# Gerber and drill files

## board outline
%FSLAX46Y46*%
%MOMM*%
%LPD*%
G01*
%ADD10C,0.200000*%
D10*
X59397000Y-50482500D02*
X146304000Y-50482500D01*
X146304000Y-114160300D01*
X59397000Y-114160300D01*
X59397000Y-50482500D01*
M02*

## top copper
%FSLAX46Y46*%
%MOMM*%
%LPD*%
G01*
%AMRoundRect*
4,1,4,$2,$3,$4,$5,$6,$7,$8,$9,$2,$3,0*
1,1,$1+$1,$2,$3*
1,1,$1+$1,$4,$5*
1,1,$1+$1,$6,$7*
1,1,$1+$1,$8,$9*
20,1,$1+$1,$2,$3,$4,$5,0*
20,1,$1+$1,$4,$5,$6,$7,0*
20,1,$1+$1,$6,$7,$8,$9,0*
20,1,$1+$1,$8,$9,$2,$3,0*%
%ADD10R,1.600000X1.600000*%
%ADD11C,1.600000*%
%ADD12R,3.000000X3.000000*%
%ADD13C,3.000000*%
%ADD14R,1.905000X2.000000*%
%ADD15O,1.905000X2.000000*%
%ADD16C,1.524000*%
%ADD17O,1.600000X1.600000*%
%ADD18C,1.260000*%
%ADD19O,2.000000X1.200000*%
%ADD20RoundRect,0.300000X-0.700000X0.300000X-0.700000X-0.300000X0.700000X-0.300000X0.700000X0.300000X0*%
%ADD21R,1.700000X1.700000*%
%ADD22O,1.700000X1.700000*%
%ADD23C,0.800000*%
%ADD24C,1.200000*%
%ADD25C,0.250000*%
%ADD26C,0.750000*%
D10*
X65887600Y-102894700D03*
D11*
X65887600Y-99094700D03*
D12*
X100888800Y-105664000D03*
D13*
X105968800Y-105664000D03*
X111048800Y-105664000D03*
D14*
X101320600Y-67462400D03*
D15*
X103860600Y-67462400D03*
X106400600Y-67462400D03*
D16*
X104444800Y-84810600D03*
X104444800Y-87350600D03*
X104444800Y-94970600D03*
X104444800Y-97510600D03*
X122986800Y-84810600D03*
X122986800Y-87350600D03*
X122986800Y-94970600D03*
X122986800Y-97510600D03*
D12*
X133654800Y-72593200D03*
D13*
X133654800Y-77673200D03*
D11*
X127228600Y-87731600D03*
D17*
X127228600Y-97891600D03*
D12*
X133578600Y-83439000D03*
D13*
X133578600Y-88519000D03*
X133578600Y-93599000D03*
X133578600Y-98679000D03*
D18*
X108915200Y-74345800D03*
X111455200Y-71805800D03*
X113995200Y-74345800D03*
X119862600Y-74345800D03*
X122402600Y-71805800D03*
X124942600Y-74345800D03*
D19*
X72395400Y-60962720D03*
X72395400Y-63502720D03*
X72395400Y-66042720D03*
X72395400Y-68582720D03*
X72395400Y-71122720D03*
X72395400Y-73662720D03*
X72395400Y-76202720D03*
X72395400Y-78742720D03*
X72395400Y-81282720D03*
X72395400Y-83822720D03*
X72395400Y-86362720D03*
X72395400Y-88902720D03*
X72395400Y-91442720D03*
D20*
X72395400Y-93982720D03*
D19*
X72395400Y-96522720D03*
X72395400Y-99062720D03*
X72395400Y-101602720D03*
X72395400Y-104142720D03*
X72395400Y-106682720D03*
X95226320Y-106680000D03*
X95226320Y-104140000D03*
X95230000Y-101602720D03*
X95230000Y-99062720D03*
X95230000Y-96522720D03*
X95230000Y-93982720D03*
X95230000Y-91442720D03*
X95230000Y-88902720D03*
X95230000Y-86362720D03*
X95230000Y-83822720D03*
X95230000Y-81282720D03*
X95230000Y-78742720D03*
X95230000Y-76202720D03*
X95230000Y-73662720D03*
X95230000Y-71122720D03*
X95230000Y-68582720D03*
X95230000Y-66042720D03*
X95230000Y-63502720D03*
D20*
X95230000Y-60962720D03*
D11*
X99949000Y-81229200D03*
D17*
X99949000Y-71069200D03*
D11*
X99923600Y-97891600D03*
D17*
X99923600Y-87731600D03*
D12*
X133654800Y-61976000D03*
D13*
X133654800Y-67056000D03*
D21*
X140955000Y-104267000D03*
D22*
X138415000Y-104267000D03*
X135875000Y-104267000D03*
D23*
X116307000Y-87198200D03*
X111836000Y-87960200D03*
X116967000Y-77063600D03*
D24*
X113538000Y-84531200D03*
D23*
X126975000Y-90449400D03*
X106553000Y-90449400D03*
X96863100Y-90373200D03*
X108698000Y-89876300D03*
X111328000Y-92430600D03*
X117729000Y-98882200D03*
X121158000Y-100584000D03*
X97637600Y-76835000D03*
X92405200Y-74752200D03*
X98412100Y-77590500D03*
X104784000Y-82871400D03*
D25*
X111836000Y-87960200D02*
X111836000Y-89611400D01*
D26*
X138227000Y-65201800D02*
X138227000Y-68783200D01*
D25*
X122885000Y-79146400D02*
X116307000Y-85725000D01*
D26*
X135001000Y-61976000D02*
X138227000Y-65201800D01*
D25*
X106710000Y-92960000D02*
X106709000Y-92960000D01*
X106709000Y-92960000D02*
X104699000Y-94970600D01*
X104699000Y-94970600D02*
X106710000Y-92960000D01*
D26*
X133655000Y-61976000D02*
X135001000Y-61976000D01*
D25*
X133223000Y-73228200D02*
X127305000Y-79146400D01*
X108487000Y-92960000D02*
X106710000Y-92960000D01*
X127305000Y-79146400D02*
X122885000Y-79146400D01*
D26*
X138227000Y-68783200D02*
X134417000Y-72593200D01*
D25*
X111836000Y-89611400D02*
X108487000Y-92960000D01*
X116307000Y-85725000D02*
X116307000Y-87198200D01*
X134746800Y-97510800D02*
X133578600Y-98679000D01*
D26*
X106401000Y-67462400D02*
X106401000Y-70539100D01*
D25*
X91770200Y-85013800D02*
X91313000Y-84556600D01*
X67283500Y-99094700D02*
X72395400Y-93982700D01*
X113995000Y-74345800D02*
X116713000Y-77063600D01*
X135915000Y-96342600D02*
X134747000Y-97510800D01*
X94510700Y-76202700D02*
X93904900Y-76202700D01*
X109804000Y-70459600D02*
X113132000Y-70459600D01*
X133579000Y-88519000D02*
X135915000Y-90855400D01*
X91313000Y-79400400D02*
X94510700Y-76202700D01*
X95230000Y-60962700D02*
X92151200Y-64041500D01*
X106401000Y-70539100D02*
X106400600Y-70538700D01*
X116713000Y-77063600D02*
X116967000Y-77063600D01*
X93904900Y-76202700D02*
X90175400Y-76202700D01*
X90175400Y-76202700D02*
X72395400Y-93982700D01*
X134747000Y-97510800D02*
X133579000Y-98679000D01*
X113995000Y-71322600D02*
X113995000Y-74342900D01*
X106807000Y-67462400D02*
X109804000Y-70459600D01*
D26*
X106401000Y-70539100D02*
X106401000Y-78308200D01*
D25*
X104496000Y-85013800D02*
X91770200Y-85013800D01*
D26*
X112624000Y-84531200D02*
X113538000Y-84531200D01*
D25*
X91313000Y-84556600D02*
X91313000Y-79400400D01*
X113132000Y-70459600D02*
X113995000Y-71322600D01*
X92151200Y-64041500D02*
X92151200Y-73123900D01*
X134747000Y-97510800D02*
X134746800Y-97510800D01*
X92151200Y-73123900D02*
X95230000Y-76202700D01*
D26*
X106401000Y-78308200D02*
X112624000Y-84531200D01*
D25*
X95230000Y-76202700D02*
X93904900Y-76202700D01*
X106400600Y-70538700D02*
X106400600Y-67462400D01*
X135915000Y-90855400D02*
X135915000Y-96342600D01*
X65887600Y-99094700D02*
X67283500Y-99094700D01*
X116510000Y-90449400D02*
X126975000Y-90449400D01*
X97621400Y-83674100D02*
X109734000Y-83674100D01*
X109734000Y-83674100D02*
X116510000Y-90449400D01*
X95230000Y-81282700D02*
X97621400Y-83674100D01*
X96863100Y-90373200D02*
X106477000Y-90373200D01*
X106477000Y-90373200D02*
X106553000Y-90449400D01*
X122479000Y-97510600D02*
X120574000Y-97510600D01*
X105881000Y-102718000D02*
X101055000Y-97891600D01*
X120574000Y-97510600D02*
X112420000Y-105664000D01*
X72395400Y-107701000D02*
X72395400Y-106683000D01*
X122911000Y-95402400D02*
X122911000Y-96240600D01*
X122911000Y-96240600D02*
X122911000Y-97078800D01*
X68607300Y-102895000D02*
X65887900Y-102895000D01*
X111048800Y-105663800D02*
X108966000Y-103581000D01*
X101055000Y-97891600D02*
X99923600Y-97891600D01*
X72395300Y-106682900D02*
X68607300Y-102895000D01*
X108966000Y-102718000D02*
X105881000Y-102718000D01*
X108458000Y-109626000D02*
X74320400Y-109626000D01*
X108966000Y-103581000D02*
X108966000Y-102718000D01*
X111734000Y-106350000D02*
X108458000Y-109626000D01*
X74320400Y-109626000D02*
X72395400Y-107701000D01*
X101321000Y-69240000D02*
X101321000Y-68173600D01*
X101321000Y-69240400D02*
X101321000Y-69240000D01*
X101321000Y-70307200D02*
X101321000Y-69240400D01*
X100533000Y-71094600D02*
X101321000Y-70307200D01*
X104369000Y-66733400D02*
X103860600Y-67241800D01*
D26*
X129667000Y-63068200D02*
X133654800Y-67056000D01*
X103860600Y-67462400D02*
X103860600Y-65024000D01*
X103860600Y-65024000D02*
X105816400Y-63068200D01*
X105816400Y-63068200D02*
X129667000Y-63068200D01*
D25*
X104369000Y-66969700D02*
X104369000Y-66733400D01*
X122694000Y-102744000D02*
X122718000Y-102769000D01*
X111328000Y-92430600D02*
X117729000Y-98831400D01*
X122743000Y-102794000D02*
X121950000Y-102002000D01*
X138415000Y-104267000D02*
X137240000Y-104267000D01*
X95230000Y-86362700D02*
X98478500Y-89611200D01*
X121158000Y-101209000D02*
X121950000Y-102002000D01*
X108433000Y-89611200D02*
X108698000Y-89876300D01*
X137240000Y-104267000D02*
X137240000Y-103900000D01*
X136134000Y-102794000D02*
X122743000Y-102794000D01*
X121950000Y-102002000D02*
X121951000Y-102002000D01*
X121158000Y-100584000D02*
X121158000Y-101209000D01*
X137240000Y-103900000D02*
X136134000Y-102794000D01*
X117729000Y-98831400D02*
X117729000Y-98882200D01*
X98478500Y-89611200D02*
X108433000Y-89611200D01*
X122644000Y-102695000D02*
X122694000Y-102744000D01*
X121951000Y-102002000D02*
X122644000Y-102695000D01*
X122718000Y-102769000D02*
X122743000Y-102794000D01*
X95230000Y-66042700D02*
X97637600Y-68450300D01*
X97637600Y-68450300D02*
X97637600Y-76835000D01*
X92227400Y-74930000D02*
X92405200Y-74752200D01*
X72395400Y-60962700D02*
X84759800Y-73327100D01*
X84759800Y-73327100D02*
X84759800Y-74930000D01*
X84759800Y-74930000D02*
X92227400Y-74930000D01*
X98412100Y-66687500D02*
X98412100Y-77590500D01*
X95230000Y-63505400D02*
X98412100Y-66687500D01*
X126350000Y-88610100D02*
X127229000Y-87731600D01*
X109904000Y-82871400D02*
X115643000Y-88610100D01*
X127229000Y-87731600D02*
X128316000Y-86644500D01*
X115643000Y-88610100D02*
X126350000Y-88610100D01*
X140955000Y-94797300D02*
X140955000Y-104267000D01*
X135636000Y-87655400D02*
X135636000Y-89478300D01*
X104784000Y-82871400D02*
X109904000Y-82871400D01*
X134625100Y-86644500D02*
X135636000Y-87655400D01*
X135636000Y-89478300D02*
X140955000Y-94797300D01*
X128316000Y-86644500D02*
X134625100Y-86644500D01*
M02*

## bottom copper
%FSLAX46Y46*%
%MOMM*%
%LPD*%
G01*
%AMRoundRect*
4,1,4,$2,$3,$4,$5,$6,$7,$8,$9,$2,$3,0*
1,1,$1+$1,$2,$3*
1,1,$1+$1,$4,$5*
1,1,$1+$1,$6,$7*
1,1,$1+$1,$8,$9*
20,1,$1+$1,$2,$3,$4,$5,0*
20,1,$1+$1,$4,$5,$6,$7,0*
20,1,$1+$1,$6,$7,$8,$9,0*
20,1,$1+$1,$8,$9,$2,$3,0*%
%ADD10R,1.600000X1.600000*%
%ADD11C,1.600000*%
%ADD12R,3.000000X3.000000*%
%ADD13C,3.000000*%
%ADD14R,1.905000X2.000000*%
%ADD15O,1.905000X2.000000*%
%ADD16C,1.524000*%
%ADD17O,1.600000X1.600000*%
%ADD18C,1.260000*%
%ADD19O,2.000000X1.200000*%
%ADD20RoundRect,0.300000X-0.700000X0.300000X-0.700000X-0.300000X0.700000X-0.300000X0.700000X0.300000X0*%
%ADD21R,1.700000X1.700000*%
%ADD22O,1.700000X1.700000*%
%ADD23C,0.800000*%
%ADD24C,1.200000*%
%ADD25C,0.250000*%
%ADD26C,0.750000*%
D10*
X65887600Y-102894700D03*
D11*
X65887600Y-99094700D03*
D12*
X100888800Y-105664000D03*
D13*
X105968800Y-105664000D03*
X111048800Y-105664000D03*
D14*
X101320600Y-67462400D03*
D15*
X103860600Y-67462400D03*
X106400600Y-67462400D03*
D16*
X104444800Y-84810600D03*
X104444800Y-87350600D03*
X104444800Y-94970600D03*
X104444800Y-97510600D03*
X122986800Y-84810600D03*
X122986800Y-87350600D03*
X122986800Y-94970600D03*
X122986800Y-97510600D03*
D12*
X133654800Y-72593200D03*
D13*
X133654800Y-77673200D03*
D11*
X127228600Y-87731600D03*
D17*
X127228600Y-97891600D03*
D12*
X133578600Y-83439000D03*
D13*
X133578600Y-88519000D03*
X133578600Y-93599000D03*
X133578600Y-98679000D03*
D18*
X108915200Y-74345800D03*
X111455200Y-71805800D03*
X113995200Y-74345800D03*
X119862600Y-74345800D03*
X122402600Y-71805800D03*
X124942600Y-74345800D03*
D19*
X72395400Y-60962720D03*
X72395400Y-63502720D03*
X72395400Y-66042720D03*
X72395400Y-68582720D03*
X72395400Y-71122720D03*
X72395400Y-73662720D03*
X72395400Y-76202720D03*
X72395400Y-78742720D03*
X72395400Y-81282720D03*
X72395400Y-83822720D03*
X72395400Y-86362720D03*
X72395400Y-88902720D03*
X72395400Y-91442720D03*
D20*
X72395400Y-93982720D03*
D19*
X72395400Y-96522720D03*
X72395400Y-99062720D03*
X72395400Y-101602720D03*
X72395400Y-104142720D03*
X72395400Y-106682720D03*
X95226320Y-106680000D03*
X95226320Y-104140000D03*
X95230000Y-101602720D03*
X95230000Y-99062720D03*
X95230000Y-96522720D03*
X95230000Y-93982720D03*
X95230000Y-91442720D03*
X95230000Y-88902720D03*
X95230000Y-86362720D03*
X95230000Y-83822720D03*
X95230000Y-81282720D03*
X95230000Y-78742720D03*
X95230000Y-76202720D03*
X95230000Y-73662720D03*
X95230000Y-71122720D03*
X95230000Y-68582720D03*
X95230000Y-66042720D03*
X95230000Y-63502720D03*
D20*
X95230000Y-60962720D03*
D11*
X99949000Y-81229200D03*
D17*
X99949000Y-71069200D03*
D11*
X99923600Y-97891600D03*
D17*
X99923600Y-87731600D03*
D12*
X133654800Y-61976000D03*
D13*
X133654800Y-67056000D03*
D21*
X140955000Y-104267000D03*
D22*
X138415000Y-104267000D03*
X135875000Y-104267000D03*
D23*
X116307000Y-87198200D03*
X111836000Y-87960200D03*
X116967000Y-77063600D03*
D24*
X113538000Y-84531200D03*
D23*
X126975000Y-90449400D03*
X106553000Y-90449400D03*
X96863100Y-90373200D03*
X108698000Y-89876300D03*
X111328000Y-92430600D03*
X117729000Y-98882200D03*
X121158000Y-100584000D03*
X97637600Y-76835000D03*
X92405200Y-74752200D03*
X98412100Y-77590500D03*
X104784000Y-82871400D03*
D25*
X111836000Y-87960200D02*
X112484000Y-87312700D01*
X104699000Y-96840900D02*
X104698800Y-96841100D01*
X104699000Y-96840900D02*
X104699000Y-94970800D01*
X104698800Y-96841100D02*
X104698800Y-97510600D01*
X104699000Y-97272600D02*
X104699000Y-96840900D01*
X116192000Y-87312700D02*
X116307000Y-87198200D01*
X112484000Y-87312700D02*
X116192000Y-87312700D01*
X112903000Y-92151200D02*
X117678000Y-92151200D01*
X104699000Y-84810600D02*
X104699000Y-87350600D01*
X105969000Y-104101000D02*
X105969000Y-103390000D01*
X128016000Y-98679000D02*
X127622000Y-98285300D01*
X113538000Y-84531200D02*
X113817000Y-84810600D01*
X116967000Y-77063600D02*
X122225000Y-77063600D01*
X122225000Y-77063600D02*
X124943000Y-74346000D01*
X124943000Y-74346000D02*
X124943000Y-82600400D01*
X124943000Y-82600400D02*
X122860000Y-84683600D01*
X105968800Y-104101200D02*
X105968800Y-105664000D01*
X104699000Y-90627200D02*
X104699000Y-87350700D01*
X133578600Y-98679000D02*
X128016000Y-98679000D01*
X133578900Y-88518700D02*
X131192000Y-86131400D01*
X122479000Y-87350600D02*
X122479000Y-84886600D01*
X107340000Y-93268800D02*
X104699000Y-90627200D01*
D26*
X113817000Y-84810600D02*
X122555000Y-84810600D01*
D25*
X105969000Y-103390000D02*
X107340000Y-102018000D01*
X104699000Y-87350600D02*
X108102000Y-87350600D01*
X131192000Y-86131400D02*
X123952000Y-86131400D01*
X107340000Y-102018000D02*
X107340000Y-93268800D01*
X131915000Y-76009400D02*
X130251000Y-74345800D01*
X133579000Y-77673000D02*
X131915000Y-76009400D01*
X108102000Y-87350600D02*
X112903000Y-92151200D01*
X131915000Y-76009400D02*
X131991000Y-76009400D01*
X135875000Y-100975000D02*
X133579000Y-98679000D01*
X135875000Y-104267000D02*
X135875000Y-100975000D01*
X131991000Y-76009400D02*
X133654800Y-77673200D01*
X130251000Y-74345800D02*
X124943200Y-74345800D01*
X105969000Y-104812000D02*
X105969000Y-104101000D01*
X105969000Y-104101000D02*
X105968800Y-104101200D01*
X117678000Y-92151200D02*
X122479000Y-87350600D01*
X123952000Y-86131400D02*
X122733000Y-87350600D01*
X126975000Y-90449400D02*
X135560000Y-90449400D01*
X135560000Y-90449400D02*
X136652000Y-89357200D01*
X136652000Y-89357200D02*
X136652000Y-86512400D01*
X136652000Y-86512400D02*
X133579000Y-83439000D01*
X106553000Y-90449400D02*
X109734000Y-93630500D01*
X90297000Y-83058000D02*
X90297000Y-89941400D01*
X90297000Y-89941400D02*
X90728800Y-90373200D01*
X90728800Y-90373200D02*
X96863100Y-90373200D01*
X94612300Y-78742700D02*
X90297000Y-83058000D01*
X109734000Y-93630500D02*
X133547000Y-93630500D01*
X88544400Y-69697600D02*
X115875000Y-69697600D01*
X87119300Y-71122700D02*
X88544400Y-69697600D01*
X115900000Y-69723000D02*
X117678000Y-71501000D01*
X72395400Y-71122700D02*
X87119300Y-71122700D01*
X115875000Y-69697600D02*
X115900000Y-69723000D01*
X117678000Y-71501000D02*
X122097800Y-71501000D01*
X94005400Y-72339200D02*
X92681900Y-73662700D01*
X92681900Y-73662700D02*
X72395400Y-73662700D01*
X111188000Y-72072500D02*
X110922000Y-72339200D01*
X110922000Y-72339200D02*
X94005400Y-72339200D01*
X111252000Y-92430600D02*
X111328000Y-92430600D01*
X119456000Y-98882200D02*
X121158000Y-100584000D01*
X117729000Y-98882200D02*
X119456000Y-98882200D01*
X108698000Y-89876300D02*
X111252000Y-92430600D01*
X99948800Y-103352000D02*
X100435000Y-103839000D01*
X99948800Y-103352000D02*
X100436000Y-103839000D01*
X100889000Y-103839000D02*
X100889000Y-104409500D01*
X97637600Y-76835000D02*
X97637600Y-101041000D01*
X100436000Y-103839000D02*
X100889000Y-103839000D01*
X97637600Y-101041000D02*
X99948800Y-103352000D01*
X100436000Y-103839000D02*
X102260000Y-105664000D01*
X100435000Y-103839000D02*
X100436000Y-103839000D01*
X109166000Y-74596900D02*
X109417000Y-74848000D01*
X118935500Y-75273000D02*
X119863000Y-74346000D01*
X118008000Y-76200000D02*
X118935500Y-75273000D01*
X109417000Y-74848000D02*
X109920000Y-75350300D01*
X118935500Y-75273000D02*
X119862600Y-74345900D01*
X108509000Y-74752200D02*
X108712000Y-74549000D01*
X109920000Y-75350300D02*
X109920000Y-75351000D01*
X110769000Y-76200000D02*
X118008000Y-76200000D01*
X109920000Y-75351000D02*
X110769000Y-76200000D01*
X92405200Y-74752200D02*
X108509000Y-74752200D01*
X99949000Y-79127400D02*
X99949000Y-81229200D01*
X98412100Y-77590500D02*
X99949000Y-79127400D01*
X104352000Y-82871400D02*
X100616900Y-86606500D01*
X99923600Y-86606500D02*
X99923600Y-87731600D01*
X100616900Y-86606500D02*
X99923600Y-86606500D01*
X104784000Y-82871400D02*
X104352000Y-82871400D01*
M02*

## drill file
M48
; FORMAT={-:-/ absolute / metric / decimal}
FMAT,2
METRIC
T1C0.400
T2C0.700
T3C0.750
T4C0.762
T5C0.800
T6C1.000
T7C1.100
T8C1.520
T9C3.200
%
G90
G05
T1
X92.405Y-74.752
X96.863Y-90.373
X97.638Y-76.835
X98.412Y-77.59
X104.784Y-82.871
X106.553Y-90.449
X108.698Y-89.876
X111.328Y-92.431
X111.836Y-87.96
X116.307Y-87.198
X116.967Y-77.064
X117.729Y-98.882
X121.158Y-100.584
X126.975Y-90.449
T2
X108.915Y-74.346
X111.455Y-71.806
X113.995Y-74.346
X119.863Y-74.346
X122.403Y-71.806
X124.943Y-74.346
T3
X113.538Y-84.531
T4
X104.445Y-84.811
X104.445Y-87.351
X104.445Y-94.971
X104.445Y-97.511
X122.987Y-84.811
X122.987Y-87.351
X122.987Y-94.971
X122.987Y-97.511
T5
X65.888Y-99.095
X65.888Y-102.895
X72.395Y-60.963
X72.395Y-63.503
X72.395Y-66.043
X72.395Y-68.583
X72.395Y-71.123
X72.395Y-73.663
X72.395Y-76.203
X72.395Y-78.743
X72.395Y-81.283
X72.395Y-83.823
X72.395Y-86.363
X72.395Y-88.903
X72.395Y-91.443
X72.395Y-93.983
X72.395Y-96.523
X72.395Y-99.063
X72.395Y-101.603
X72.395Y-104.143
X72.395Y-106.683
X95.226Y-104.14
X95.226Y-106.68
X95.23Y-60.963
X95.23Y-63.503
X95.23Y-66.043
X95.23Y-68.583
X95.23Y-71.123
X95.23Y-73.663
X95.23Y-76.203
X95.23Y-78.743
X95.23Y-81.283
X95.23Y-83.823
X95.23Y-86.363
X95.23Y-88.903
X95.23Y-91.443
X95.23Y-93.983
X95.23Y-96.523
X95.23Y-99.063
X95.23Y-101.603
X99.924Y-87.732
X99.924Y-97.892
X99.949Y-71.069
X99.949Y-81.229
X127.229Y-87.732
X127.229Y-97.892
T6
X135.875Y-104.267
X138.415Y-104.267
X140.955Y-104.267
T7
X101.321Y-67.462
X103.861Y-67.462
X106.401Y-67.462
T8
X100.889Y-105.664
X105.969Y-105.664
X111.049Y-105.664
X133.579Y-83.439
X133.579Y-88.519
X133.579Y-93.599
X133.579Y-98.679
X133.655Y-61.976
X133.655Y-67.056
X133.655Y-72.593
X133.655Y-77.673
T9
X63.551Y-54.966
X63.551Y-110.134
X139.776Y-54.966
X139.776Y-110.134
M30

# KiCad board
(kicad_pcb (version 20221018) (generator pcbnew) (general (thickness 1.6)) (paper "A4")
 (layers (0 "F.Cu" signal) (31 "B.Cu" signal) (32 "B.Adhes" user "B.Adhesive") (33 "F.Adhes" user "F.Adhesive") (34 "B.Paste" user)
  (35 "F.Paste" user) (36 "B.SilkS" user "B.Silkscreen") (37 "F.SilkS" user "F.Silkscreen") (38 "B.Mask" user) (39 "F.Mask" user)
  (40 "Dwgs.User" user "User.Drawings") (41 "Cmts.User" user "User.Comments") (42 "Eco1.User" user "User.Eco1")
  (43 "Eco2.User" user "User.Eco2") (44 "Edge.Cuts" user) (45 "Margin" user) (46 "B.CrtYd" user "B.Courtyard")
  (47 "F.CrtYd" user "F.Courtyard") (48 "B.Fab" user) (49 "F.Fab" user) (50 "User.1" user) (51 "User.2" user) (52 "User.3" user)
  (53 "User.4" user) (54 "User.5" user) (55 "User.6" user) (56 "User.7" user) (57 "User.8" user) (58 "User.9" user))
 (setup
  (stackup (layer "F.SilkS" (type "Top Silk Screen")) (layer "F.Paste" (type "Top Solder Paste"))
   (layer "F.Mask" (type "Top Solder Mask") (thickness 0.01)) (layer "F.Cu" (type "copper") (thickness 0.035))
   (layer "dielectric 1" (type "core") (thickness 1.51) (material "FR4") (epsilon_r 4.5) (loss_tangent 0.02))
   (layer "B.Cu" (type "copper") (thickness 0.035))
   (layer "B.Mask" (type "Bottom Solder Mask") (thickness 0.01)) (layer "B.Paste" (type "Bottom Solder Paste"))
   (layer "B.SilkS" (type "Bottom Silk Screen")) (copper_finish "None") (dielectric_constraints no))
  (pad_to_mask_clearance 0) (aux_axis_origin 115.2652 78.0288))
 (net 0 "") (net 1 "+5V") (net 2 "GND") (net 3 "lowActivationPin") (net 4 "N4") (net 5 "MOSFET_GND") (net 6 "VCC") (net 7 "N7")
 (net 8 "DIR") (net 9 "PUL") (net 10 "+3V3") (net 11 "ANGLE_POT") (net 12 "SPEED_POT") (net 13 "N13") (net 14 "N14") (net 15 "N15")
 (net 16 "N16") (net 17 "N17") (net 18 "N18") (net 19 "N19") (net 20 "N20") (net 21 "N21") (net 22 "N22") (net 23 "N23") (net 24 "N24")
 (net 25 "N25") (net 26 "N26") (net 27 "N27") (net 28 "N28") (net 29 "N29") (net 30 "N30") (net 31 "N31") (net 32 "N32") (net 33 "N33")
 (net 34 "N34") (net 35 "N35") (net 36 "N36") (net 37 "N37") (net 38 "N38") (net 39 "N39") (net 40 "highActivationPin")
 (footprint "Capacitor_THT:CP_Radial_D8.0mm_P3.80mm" (layer "F.Cu") (at 65.8876 102.8947 90)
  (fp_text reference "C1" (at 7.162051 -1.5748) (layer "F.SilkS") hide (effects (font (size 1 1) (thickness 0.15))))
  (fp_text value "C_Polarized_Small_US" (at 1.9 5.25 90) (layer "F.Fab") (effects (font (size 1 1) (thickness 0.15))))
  (pad "1" thru_hole rect (at 0 0 90) (size 1.6 1.6) (drill 0.8) (layers "*.Cu" "*.Mask") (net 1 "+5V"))
  (pad "2" thru_hole circle (at 3.8 0 90) (size 1.6 1.6) (drill 0.8) (layers "*.Cu" "*.Mask") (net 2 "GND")))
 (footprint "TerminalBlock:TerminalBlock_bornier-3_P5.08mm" (layer "F.Cu") (at 100.8888 105.664)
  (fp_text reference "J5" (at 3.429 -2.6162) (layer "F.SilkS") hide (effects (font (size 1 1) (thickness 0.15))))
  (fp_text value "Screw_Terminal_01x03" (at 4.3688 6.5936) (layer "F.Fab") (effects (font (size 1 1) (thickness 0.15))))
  (pad "1" thru_hole rect (at 0 0) (size 3 3) (drill 1.52) (layers "*.Cu" "*.Mask") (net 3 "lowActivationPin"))
  (pad "2" thru_hole circle (at 5.08 0) (size 3 3) (drill 1.52) (layers "*.Cu" "*.Mask") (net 2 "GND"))
  (pad "3" thru_hole circle (at 10.16 0) (size 3 3) (drill 1.52) (layers "*.Cu" "*.Mask") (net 1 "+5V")))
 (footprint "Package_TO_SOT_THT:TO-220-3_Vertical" (layer "F.Cu") (at 101.3206 67.4624)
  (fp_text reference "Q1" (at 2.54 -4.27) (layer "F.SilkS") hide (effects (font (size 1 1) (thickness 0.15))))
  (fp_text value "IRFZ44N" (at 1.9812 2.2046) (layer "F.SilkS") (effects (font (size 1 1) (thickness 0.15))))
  (pad "1" thru_hole rect (at 0 0) (size 1.905 2) (drill 1.1) (layers "*.Cu" "*.Mask") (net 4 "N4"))
  (pad "2" thru_hole oval (at 2.54 0) (size 1.905 2) (drill 1.1) (layers "*.Cu" "*.Mask") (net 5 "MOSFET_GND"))
  (pad "3" thru_hole oval (at 5.08 0) (size 1.905 2) (drill 1.1) (layers "*.Cu" "*.Mask") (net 2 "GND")))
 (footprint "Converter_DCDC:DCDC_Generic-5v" (layer "F.Cu") (at 114.8588 92.4306)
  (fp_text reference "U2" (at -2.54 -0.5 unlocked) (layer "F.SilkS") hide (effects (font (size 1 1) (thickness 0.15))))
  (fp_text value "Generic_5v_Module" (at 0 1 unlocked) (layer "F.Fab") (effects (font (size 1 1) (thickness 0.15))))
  (pad "1" thru_hole circle (at -10.414 -7.62) (size 1.524 1.524) (drill 0.762) (layers "*.Cu" "*.Mask") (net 2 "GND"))
  (pad "1" thru_hole circle (at -10.414 -5.08) (size 1.524 1.524) (drill 0.762) (layers "*.Cu" "*.Mask") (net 2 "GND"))
  (pad "2" thru_hole circle (at -10.414 2.54) (size 1.524 1.524) (drill 0.762) (layers "*.Cu" "*.Mask") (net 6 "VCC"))
  (pad "2" thru_hole circle (at -10.414 5.08) (size 1.524 1.524) (drill 0.762) (layers "*.Cu" "*.Mask") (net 6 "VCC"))
  (pad "3" thru_hole circle (at 8.128 -7.62) (size 1.524 1.524) (drill 0.762) (layers "*.Cu" "*.Mask") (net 2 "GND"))
  (pad "3" thru_hole circle (at 8.128 -5.08) (size 1.524 1.524) (drill 0.762) (layers "*.Cu" "*.Mask") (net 2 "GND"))
  (pad "4" thru_hole circle (at 8.128 2.54) (size 1.524 1.524) (drill 0.762) (layers "*.Cu" "*.Mask") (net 1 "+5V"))
  (pad "4" thru_hole circle (at 8.128 5.08) (size 1.524 1.524) (drill 0.762) (layers "*.Cu" "*.Mask") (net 1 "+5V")))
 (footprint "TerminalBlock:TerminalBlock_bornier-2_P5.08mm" (layer "F.Cu") (at 133.6548 72.5932 -90)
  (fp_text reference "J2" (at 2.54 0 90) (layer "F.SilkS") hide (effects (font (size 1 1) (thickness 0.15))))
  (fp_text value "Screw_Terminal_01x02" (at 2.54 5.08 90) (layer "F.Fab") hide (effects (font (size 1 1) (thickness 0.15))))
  (pad "1" thru_hole rect (at 0 0 270) (size 3 3) (drill 1.52) (layers "*.Cu" "*.Mask") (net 6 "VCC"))
  (pad "2" thru_hole circle (at 5.08 0 270) (size 3 3) (drill 1.52) (layers "*.Cu" "*.Mask") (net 2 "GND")))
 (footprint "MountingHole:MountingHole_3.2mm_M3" (layer "F.Cu") (at 63.5508 54.9656)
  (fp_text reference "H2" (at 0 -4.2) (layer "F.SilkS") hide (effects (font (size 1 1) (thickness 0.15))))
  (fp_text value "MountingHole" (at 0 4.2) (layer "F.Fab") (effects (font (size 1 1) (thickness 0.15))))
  (pad "" np_thru_hole circle (at 0 0) (size 3.2 3.2) (drill 3.2) (layers "F&B.Cu" "*.Mask")))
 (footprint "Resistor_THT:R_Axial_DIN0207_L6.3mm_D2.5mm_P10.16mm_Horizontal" (layer "F.Cu") (at 127.2286 87.7316 -90)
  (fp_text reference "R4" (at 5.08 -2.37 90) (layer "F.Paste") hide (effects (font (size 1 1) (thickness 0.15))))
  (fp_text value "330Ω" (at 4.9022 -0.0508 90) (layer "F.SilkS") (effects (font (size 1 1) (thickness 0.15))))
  (pad "1" thru_hole circle (at 0 0 270) (size 1.6 1.6) (drill 0.8) (layers "*.Cu" "*.Mask") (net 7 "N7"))
  (pad "2" thru_hole oval (at 10.16 0 270) (size 1.6 1.6) (drill 0.8) (layers "*.Cu" "*.Mask") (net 2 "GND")))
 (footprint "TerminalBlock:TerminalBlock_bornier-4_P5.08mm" (layer "F.Cu") (at 133.5786 83.439 -90)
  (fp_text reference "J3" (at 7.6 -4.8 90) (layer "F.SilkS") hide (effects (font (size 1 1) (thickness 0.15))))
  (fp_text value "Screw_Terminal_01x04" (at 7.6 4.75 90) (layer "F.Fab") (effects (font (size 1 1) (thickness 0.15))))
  (pad "1" thru_hole rect (at 0 0 270) (size 3 3) (drill 1.52) (layers "*.Cu" "*.Mask") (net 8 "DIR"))
  (pad "2" thru_hole circle (at 5.08 0 270) (size 3 3) (drill 1.52) (layers "*.Cu" "*.Mask") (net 2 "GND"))
  (pad "3" thru_hole circle (at 10.16 0 270) (size 3 3) (drill 1.52) (layers "*.Cu" "*.Mask") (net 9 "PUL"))
  (pad "4" thru_hole circle (at 15.24 0 270) (size 3 3) (drill 1.52) (layers "*.Cu" "*.Mask") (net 2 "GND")))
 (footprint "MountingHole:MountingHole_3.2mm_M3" (layer "F.Cu") (at 139.6492 110.0328)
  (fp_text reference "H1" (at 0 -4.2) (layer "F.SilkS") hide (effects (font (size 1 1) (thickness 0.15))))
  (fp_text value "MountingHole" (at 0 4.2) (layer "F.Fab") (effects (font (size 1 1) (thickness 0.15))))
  (pad "" np_thru_hole circle (at 0.127 0.1016) (size 3.2 3.2) (drill 3.2) (layers "F&B.Cu" "*.Mask")))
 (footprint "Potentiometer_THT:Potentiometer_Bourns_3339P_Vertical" (layer "F.Cu") (at 108.9152 74.3458 -90)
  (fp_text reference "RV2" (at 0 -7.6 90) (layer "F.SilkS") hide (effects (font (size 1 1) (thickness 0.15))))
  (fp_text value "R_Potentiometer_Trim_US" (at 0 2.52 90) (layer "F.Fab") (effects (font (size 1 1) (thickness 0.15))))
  (pad "1" thru_hole circle (at 0 0 270) (size 1.26 1.26) (drill 0.7) (layers "*.Cu" "*.Mask") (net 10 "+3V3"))
  (pad "2" thru_hole circle (at -2.54 -2.54 270) (size 1.26 1.26) (drill 0.7) (layers "*.Cu" "*.Mask") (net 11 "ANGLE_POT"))
  (pad "3" thru_hole circle (at 0 -5.08 270) (size 1.26 1.26) (drill 0.7) (layers "*.Cu" "*.Mask") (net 2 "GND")))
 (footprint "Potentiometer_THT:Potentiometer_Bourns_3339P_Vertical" (layer "F.Cu") (at 119.8626 74.3458 -90)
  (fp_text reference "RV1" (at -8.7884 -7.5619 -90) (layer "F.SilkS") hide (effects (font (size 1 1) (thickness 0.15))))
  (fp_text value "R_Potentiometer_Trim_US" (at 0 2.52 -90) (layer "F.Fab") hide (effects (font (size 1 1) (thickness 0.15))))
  (pad "1" thru_hole circle (at 0 0 270) (size 1.26 1.26) (drill 0.7) (layers "*.Cu" "*.Mask") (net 10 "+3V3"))
  (pad "2" thru_hole circle (at -2.54 -2.54 270) (size 1.26 1.26) (drill 0.7) (layers "*.Cu" "*.Mask") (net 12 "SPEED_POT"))
  (pad "3" thru_hole circle (at 0 -5.08 270) (size 1.26 1.26) (drill 0.7) (layers "*.Cu" "*.Mask") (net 2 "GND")))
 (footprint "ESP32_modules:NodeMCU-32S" (layer "F.Cu") (at 71.12 60.96)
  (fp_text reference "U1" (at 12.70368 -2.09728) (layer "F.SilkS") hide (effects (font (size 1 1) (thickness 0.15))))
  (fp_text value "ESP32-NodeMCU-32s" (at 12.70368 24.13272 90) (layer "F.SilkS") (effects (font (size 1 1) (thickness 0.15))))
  (pad "1" thru_hole oval (at 1.2754 0.00272 270) (size 1.2 2) (drill 0.8) (layers "*.Cu" "*.Mask") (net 10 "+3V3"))
  (pad "2" thru_hole oval (at 1.2754 2.54272 270) (size 1.2 2) (drill 0.8) (layers "*.Cu" "*.Mask") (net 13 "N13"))
  (pad "3" thru_hole oval (at 1.2754 5.08272 270) (size 1.2 2) (drill 0.8) (layers "*.Cu" "*.Mask") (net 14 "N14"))
  (pad "4" thru_hole oval (at 1.2754 7.62272 270) (size 1.2 2) (drill 0.8) (layers "*.Cu" "*.Mask") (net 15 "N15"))
  (pad "5" thru_hole oval (at 1.2754 10.16272 270) (size 1.2 2) (drill 0.8) (layers "*.Cu" "*.Mask") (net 12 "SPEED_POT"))
  (pad "6" thru_hole oval (at 1.2754 12.70272 270) (size 1.2 2) (drill 0.8) (layers "*.Cu" "*.Mask") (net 11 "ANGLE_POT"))
  (pad "7" thru_hole oval (at 1.2754 15.24272 270) (size 1.2 2) (drill 0.8) (layers "*.Cu" "*.Mask") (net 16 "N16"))
  (pad "8" thru_hole oval (at 1.2754 17.78272 270) (size 1.2 2) (drill 0.8) (layers "*.Cu" "*.Mask") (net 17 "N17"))
  (pad "9" thru_hole oval (at 1.2754 20.32272 270) (size 1.2 2) (drill 0.8) (layers "*.Cu" "*.Mask") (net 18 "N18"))
  (pad "10" thru_hole oval (at 1.2754 22.86272 270) (size 1.2 2) (drill 0.8) (layers "*.Cu" "*.Mask") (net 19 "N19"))
  (pad "11" thru_hole oval (at 1.2754 25.40272 270) (size 1.2 2) (drill 0.8) (layers "*.Cu" "*.Mask") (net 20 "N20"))
  (pad "12" thru_hole oval (at 1.2754 27.94272 270) (size 1.2 2) (drill 0.8) (layers "*.Cu" "*.Mask") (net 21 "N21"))
  (pad "13" thru_hole oval (at 1.2754 30.48272 270) (size 1.2 2) (drill 0.8) (layers "*.Cu" "*.Mask") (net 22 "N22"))
  (pad "14" thru_hole roundrect (at 1.2754 33.02272 270) (size 1.2 2) (drill 0.8) (layers "*.Cu" "*.Mask") (roundrect_rratio 0.25)
   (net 2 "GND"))
  (pad "15" thru_hole oval (at 1.2754 35.56272 270) (size 1.2 2) (drill 0.8) (layers "*.Cu" "*.Mask") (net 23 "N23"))
  (pad "16" thru_hole oval (at 1.2754 38.10272 270) (size 1.2 2) (drill 0.8) (layers "*.Cu" "*.Mask") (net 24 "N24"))
  (pad "17" thru_hole oval (at 1.2754 40.64272 270) (size 1.2 2) (drill 0.8) (layers "*.Cu" "*.Mask") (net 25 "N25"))
  (pad "18" thru_hole oval (at 1.2754 43.18272 270) (size 1.2 2) (drill 0.8) (layers "*.Cu" "*.Mask") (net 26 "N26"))
  (pad "19" thru_hole oval (at 1.2754 45.72272 270) (size 1.2 2) (drill 0.8) (layers "*.Cu" "*.Mask") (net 1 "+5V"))
  (pad "20" thru_hole oval (at 24.10632 45.72 270) (size 1.2 2) (drill 0.8) (layers "*.Cu" "*.Mask") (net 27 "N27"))
  (pad "21" thru_hole oval (at 24.10632 43.18 270) (size 1.2 2) (drill 0.8) (layers "*.Cu" "*.Mask") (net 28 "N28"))
  (pad "22" thru_hole oval (at 24.11 40.64272 270) (size 1.2 2) (drill 0.8) (layers "*.Cu" "*.Mask") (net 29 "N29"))
  (pad "23" thru_hole oval (at 24.11 38.10272 270) (size 1.2 2) (drill 0.8) (layers "*.Cu" "*.Mask") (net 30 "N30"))
  (pad "24" thru_hole oval (at 24.11 35.56272 270) (size 1.2 2) (drill 0.8) (layers "*.Cu" "*.Mask") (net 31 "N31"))
  (pad "25" thru_hole oval (at 24.11 33.02272 270) (size 1.2 2) (drill 0.8) (layers "*.Cu" "*.Mask") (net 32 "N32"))
  (pad "26" thru_hole oval (at 24.11 30.48272 270) (size 1.2 2) (drill 0.8) (layers "*.Cu" "*.Mask") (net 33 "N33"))
  (pad "27" thru_hole oval (at 24.11 27.94272 270) (size 1.2 2) (drill 0.8) (layers "*.Cu" "*.Mask") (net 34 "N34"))
  (pad "28" thru_hole oval (at 24.11 25.40272 270) (size 1.2 2) (drill 0.8) (layers "*.Cu" "*.Mask") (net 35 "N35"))
  (pad "29" thru_hole oval (at 24.11 22.86272 270) (size 1.2 2) (drill 0.8) (layers "*.Cu" "*.Mask") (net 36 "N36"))
  (pad "30" thru_hole oval (at 24.11 20.32272 270) (size 1.2 2) (drill 0.8) (layers "*.Cu" "*.Mask") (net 8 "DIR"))
  (pad "31" thru_hole oval (at 24.11 17.78272 270) (size 1.2 2) (drill 0.8) (layers "*.Cu" "*.Mask") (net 9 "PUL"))
  (pad "32" thru_hole oval (at 24.11 15.24272 270) (size 1.2 2) (drill 0.8) (layers "*.Cu" "*.Mask") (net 2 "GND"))
  (pad "33" thru_hole oval (at 24.11 12.70272 270) (size 1.2 2) (drill 0.8) (layers "*.Cu" "*.Mask") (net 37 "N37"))
  (pad "34" thru_hole oval (at 24.11 10.16272 270) (size 1.2 2) (drill 0.8) (layers "*.Cu" "*.Mask") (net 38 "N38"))
  (pad "35" thru_hole oval (at 24.11 7.62272 270) (size 1.2 2) (drill 0.8) (layers "*.Cu" "*.Mask") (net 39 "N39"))
  (pad "36" thru_hole oval (at 24.11 5.08272 270) (size 1.2 2) (drill 0.8) (layers "*.Cu" "*.Mask") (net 3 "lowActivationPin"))
  (pad "37" thru_hole oval (at 24.11 2.54272 270) (size 1.2 2) (drill 0.8) (layers "*.Cu" "*.Mask") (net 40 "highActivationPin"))
  (pad "38" thru_hole roundrect (at 24.11 0.00272 270) (size 1.2 2) (drill 0.8) (layers "*.Cu" "*.Mask") (roundrect_rratio 0.25)
   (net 2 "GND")))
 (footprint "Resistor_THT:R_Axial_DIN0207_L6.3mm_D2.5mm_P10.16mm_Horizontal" (layer "F.Cu") (at 99.949 81.2292 90)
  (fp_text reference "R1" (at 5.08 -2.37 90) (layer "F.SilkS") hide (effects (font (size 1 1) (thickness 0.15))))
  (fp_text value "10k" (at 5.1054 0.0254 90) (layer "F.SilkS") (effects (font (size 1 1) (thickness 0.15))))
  (pad "1" thru_hole circle (at 0 0 90) (size 1.6 1.6) (drill 0.8) (layers "*.Cu" "*.Mask") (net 40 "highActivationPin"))
  (pad "2" thru_hole oval (at 10.16 0 90) (size 1.6 1.6) (drill 0.8) (layers "*.Cu" "*.Mask") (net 4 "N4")))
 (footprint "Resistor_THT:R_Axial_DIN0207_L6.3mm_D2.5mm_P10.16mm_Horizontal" (layer "F.Cu") (at 99.9236 97.8916 90)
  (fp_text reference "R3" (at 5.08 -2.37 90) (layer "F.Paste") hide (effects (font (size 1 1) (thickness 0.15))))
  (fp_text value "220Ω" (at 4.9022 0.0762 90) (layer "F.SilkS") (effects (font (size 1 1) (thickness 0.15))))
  (pad "1" thru_hole circle (at 0 0 90) (size 1.6 1.6) (drill 0.8) (layers "*.Cu" "*.Mask") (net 1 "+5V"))
  (pad "2" thru_hole oval (at 10.16 0 90) (size 1.6 1.6) (drill 0.8) (layers "*.Cu" "*.Mask") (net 7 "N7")))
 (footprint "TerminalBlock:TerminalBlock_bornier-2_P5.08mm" (layer "F.Cu") (at 133.6548 61.976 -90)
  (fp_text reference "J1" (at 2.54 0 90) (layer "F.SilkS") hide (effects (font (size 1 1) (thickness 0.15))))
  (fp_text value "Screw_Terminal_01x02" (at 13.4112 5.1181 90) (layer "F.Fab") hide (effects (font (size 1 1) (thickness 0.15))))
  (pad "1" thru_hole rect (at 0 0 270) (size 3 3) (drill 1.52) (layers "*.Cu" "*.Mask") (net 6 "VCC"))
  (pad "2" thru_hole circle (at 5.08 0 270) (size 3 3) (drill 1.52) (layers "*.Cu" "*.Mask") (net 5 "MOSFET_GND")))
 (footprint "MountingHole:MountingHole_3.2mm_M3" (layer "F.Cu") (at 63.5762 110.1344)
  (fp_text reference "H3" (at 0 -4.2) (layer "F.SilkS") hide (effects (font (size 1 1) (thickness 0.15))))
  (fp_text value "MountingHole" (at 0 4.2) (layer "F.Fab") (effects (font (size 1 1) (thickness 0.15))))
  (pad "" np_thru_hole circle (at -0.0254 0) (size 3.2 3.2) (drill 3.2) (layers "F&B.Cu" "*.Mask")))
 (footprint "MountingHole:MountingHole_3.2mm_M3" (layer "F.Cu") (at 139.8778 54.991)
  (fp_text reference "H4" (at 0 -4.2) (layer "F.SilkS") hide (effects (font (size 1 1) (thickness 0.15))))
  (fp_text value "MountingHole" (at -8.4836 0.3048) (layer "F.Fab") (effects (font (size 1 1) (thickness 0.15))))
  (pad "" np_thru_hole circle (at -0.1016 -0.0254) (size 3.2 3.2) (drill 3.2) (layers "F&B.Cu" "*.Mask")))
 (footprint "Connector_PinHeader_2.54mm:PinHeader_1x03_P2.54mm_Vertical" (layer "F.Cu") (at 140.955 104.267 -90)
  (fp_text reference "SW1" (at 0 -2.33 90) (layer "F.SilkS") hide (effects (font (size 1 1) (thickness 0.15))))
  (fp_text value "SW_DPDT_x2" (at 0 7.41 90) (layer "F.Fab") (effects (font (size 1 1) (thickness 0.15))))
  (pad "1" thru_hole rect (at 0 0 270) (size 1.7 1.7) (drill 1) (layers "*.Cu" "*.Mask") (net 7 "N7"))
  (pad "2" thru_hole oval (at 0 2.54 270) (size 1.7 1.7) (drill 1) (layers "*.Cu" "*.Mask") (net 35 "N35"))
  (pad "3" thru_hole oval (at 0 5.08 270) (size 1.7 1.7) (drill 1) (layers "*.Cu" "*.Mask") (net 2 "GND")))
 (gr_rect (start 59.397 50.4825) (end 146.304 114.1603) (stroke (width 0.2) (type solid)) (fill none) (layer "Edge.Cuts"))
 (segment (start 111.836 87.9602) (end 111.836 89.6114) (width 0.25) (layer "F.Cu") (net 6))
 (segment (start 138.227 65.2018) (end 138.227 68.7832) (width 0.75) (layer "F.Cu") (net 6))
 (segment (start 122.885 79.1464) (end 116.307 85.725) (width 0.25) (layer "F.Cu") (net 6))
 (segment (start 135.001 61.976) (end 138.227 65.2018) (width 0.75) (layer "F.Cu") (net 6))
 (segment (start 106.71 92.96) (end 106.709 92.96) (width 0.25) (layer "F.Cu") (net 6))
 (segment (start 106.709 92.96) (end 104.699 94.9706) (width 0.25) (layer "F.Cu") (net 6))
 (segment (start 104.699 94.9706) (end 106.71 92.96) (width 0.25) (layer "F.Cu") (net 6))
 (segment (start 133.655 61.976) (end 135.001 61.976) (width 0.75) (layer "F.Cu") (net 6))
 (segment (start 133.223 73.2282) (end 127.305 79.1464) (width 0.25) (layer "F.Cu") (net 6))
 (segment (start 108.487 92.96) (end 106.71 92.96) (width 0.25) (layer "F.Cu") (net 6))
 (segment (start 127.305 79.1464) (end 122.885 79.1464) (width 0.25) (layer "F.Cu") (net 6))
 (segment (start 138.227 68.7832) (end 134.417 72.5932) (width 0.75) (layer "F.Cu") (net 6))
 (segment (start 111.836 89.6114) (end 108.487 92.96) (width 0.25) (layer "F.Cu") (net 6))
 (segment (start 116.307 85.725) (end 116.307 87.1982) (width 0.25) (layer "F.Cu") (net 6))
 (via (at 116.307 87.1982) (size 0.8) (drill 0.4) (layers "F.Cu" "B.Cu") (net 6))
 (via (at 111.836 87.9602) (size 0.8) (drill 0.4) (layers "F.Cu" "B.Cu") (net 6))
 (segment (start 111.836 87.9602) (end 112.484 87.3127) (width 0.25) (layer "B.Cu") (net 6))
 (segment (start 104.699 96.8409) (end 104.6988 96.8411) (width 0.25) (layer "B.Cu") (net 6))
 (segment (start 104.699 96.8409) (end 104.699 94.9708) (width 0.25) (layer "B.Cu") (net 6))
 (segment (start 104.6988 96.8411) (end 104.6988 97.5106) (width 0.25) (layer "B.Cu") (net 6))
 (segment (start 104.699 97.2726) (end 104.699 96.8409) (width 0.25) (layer "B.Cu") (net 6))
 (segment (start 116.192 87.3127) (end 116.307 87.1982) (width 0.25) (layer "B.Cu") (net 6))
 (segment (start 112.484 87.3127) (end 116.192 87.3127) (width 0.25) (layer "B.Cu") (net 6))
 (segment (start 134.7468 97.5108) (end 133.5786 98.679) (width 0.25) (layer "F.Cu") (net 2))
 (segment (start 106.401 67.4624) (end 106.401 70.5391) (width 0.75) (layer "F.Cu") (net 2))
 (segment (start 91.7702 85.0138) (end 91.313 84.5566) (width 0.25) (layer "F.Cu") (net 2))
 (segment (start 67.2835 99.0947) (end 72.3954 93.9827) (width 0.25) (layer "F.Cu") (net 2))
 (segment (start 113.995 74.3458) (end 116.713 77.0636) (width 0.25) (layer "F.Cu") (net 2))
 (segment (start 135.915 96.3426) (end 134.747 97.5108) (width 0.25) (layer "F.Cu") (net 2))
 (segment (start 94.5107 76.2027) (end 93.9049 76.2027) (width 0.25) (layer "F.Cu") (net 2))
 (segment (start 109.804 70.4596) (end 113.132 70.4596) (width 0.25) (layer "F.Cu") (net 2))
 (segment (start 133.579 88.519) (end 135.915 90.8554) (width 0.25) (layer "F.Cu") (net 2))
 (segment (start 91.313 79.4004) (end 94.5107 76.2027) (width 0.25) (layer "F.Cu") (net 2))
 (segment (start 95.23 60.9627) (end 92.1512 64.0415) (width 0.25) (layer "F.Cu") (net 2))
 (segment (start 106.401 70.5391) (end 106.4006 70.5387) (width 0.25) (layer "F.Cu") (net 2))
 (segment (start 116.713 77.0636) (end 116.967 77.0636) (width 0.25) (layer "F.Cu") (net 2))
 (segment (start 93.9049 76.2027) (end 90.1754 76.2027) (width 0.25) (layer "F.Cu") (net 2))
 (segment (start 90.1754 76.2027) (end 72.3954 93.9827) (width 0.25) (layer "F.Cu") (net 2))
 (segment (start 134.747 97.5108) (end 133.579 98.679) (width 0.25) (layer "F.Cu") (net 2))
 (segment (start 113.995 71.3226) (end 113.995 74.3429) (width 0.25) (layer "F.Cu") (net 2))
 (segment (start 106.807 67.4624) (end 109.804 70.4596) (width 0.25) (layer "F.Cu") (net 2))
 (segment (start 106.401 70.5391) (end 106.401 78.3082) (width 0.75) (layer "F.Cu") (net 2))
 (segment (start 104.496 85.0138) (end 91.7702 85.0138) (width 0.25) (layer "F.Cu") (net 2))
 (segment (start 112.624 84.5312) (end 113.538 84.5312) (width 0.75) (layer "F.Cu") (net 2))
 (segment (start 91.313 84.5566) (end 91.313 79.4004) (width 0.25) (layer "F.Cu") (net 2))
 (segment (start 113.132 70.4596) (end 113.995 71.3226) (width 0.25) (layer "F.Cu") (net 2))
 (segment (start 92.1512 64.0415) (end 92.1512 73.1239) (width 0.25) (layer "F.Cu") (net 2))
 (segment (start 134.747 97.5108) (end 134.7468 97.5108) (width 0.25) (layer "F.Cu") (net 2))
 (segment (start 92.1512 73.1239) (end 95.23 76.2027) (width 0.25) (layer "F.Cu") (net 2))
 (segment (start 106.401 78.3082) (end 112.624 84.5312) (width 0.75) (layer "F.Cu") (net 2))
 (segment (start 95.23 76.2027) (end 93.9049 76.2027) (width 0.25) (layer "F.Cu") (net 2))
 (segment (start 106.4006 70.5387) (end 106.4006 67.4624) (width 0.25) (layer "F.Cu") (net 2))
 (segment (start 135.915 90.8554) (end 135.915 96.3426) (width 0.25) (layer "F.Cu") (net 2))
 (segment (start 65.8876 99.0947) (end 67.2835 99.0947) (width 0.25) (layer "F.Cu") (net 2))
 (via (at 116.967 77.0636) (size 0.8) (drill 0.4) (layers "F.Cu" "B.Cu") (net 2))
 (via (at 113.538 84.5312) (size 1.2) (drill 0.75) (layers "F.Cu" "B.Cu") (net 2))
 (segment (start 112.903 92.1512) (end 117.678 92.1512) (width 0.25) (layer "B.Cu") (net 2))
 (segment (start 104.699 84.8106) (end 104.699 87.3506) (width 0.25) (layer "B.Cu") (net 2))
 (segment (start 105.969 104.101) (end 105.969 103.39) (width 0.25) (layer "B.Cu") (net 2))
 (segment (start 128.016 98.679) (end 127.622 98.2853) (width 0.25) (layer "B.Cu") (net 2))
 (segment (start 113.538 84.5312) (end 113.817 84.8106) (width 0.25) (layer "B.Cu") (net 2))
 (segment (start 116.967 77.0636) (end 122.225 77.0636) (width 0.25) (layer "B.Cu") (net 2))
 (segment (start 122.225 77.0636) (end 124.943 74.346) (width 0.25) (layer "B.Cu") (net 2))
 (segment (start 124.943 74.346) (end 124.943 82.6004) (width 0.25) (layer "B.Cu") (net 2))
 (segment (start 124.943 82.6004) (end 122.86 84.6836) (width 0.25) (layer "B.Cu") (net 2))
 (segment (start 105.9688 104.1012) (end 105.9688 105.664) (width 0.25) (layer "B.Cu") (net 2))
 (segment (start 104.699 90.6272) (end 104.699 87.3507) (width 0.25) (layer "B.Cu") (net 2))
 (segment (start 133.5786 98.679) (end 128.016 98.679) (width 0.25) (layer "B.Cu") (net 2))
 (segment (start 133.5789 88.5187) (end 131.192 86.1314) (width 0.25) (layer "B.Cu") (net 2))
 (segment (start 122.479 87.3506) (end 122.479 84.8866) (width 0.25) (layer "B.Cu") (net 2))
 (segment (start 107.34 93.2688) (end 104.699 90.6272) (width 0.25) (layer "B.Cu") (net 2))
 (segment (start 113.817 84.8106) (end 122.555 84.8106) (width 0.75) (layer "B.Cu") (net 2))
 (segment (start 105.969 103.39) (end 107.34 102.018) (width 0.25) (layer "B.Cu") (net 2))
 (segment (start 104.699 87.3506) (end 108.102 87.3506) (width 0.25) (layer "B.Cu") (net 2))
 (segment (start 131.192 86.1314) (end 123.952 86.1314) (width 0.25) (layer "B.Cu") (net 2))
 (segment (start 107.34 102.018) (end 107.34 93.2688) (width 0.25) (layer "B.Cu") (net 2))
 (segment (start 131.915 76.0094) (end 130.251 74.3458) (width 0.25) (layer "B.Cu") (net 2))
 (segment (start 133.579 77.673) (end 131.915 76.0094) (width 0.25) (layer "B.Cu") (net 2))
 (segment (start 108.102 87.3506) (end 112.903 92.1512) (width 0.25) (layer "B.Cu") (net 2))
 (segment (start 131.915 76.0094) (end 131.991 76.0094) (width 0.25) (layer "B.Cu") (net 2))
 (segment (start 135.875 100.975) (end 133.579 98.679) (width 0.25) (layer "B.Cu") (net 2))
 (segment (start 135.875 104.267) (end 135.875 100.975) (width 0.25) (layer "B.Cu") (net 2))
 (segment (start 131.991 76.0094) (end 133.6548 77.6732) (width 0.25) (layer "B.Cu") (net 2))
 (segment (start 130.251 74.3458) (end 124.9432 74.3458) (width 0.25) (layer "B.Cu") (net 2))
 (segment (start 105.969 104.812) (end 105.969 104.101) (width 0.25) (layer "B.Cu") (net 2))
 (segment (start 105.969 104.101) (end 105.9688 104.1012) (width 0.25) (layer "B.Cu") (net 2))
 (segment (start 117.678 92.1512) (end 122.479 87.3506) (width 0.25) (layer "B.Cu") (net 2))
 (segment (start 123.952 86.1314) (end 122.733 87.3506) (width 0.25) (layer "B.Cu") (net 2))
 (segment (start 116.51 90.4494) (end 126.975 90.4494) (width 0.25) (layer "F.Cu") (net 8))
 (segment (start 97.6214 83.6741) (end 109.734 83.6741) (width 0.25) (layer "F.Cu") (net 8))
 (segment (start 109.734 83.6741) (end 116.51 90.4494) (width 0.25) (layer "F.Cu") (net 8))
 (segment (start 95.23 81.2827) (end 97.6214 83.6741) (width 0.25) (layer "F.Cu") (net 8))
 (via (at 126.975 90.4494) (size 0.8) (drill 0.4) (layers "F.Cu" "B.Cu") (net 8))
 (segment (start 126.975 90.4494) (end 135.56 90.4494) (width 0.25) (layer "B.Cu") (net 8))
 (segment (start 135.56 90.4494) (end 136.652 89.3572) (width 0.25) (layer "B.Cu") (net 8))
 (segment (start 136.652 89.3572) (end 136.652 86.5124) (width 0.25) (layer "B.Cu") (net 8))
 (segment (start 136.652 86.5124) (end 133.579 83.439) (width 0.25) (layer "B.Cu") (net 8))
 (segment (start 96.8631 90.3732) (end 106.477 90.3732) (width 0.25) (layer "F.Cu") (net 9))
 (segment (start 106.477 90.3732) (end 106.553 90.4494) (width 0.25) (layer "F.Cu") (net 9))
 (via (at 106.553 90.4494) (size 0.8) (drill 0.4) (layers "F.Cu" "B.Cu") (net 9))
 (via (at 96.8631 90.3732) (size 0.8) (drill 0.4) (layers "F.Cu" "B.Cu") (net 9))
 (segment (start 106.553 90.4494) (end 109.734 93.6305) (width 0.25) (layer "B.Cu") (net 9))
 (segment (start 90.297 83.058) (end 90.297 89.9414) (width 0.25) (layer "B.Cu") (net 9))
 (segment (start 90.297 89.9414) (end 90.7288 90.3732) (width 0.25) (layer "B.Cu") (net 9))
 (segment (start 90.7288 90.3732) (end 96.8631 90.3732) (width 0.25) (layer "B.Cu") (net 9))
 (segment (start 94.6123 78.7427) (end 90.297 83.058) (width 0.25) (layer "B.Cu") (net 9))
 (segment (start 109.734 93.6305) (end 133.547 93.6305) (width 0.25) (layer "B.Cu") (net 9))
 (segment (start 122.479 97.5106) (end 120.574 97.5106) (width 0.25) (layer "F.Cu") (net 1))
 (segment (start 105.881 102.718) (end 101.055 97.8916) (width 0.25) (layer "F.Cu") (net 1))
 (segment (start 120.574 97.5106) (end 112.42 105.664) (width 0.25) (layer "F.Cu") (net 1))
 (segment (start 72.3954 107.701) (end 72.3954 106.683) (width 0.25) (layer "F.Cu") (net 1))
 (segment (start 122.911 95.4024) (end 122.911 96.2406) (width 0.25) (layer "F.Cu") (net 1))
 (segment (start 122.911 96.2406) (end 122.911 97.0788) (width 0.25) (layer "F.Cu") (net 1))
 (segment (start 68.6073 102.895) (end 65.8879 102.895) (width 0.25) (layer "F.Cu") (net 1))
 (segment (start 111.0488 105.6638) (end 108.966 103.581) (width 0.25) (layer "F.Cu") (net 1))
 (segment (start 101.055 97.8916) (end 99.9236 97.8916) (width 0.25) (layer "F.Cu") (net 1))
 (segment (start 72.3953 106.6829) (end 68.6073 102.895) (width 0.25) (layer "F.Cu") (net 1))
 (segment (start 108.966 102.718) (end 105.881 102.718) (width 0.25) (layer "F.Cu") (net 1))
 (segment (start 108.458 109.626) (end 74.3204 109.626) (width 0.25) (layer "F.Cu") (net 1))
 (segment (start 108.966 103.581) (end 108.966 102.718) (width 0.25) (layer "F.Cu") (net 1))
 (segment (start 111.734 106.35) (end 108.458 109.626) (width 0.25) (layer "F.Cu") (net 1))
 (segment (start 74.3204 109.626) (end 72.3954 107.701) (width 0.25) (layer "F.Cu") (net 1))
 (segment (start 101.321 69.24) (end 101.321 68.1736) (width 0.25) (layer "F.Cu") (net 4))
 (segment (start 101.321 69.2404) (end 101.321 69.24) (width 0.25) (layer "F.Cu") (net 4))
 (segment (start 101.321 70.3072) (end 101.321 69.2404) (width 0.25) (layer "F.Cu") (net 4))
 (segment (start 100.533 71.0946) (end 101.321 70.3072) (width 0.25) (layer "F.Cu") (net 4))
 (segment (start 104.369 66.7334) (end 103.8606 67.2418) (width 0.25) (layer "F.Cu") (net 5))
 (segment (start 129.667 63.0682) (end 133.6548 67.056) (width 0.75) (layer "F.Cu") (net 5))
 (segment (start 103.8606 67.4624) (end 103.8606 65.024) (width 0.75) (layer "F.Cu") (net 5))
 (segment (start 103.8606 65.024) (end 105.8164 63.0682) (width 0.75) (layer "F.Cu") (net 5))
 (segment (start 105.8164 63.0682) (end 129.667 63.0682) (width 0.75) (layer "F.Cu") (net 5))
 (segment (start 104.369 66.9697) (end 104.369 66.7334) (width 0.25) (layer "F.Cu") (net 5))
 (segment (start 88.5444 69.6976) (end 115.875 69.6976) (width 0.25) (layer "B.Cu") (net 12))
 (segment (start 87.1193 71.1227) (end 88.5444 69.6976) (width 0.25) (layer "B.Cu") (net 12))
 (segment (start 115.9 69.723) (end 117.678 71.501) (width 0.25) (layer "B.Cu") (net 12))
 (segment (start 72.3954 71.1227) (end 87.1193 71.1227) (width 0.25) (layer "B.Cu") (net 12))
 (segment (start 115.875 69.6976) (end 115.9 69.723) (width 0.25) (layer "B.Cu") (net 12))
 (segment (start 117.678 71.501) (end 122.0978 71.501) (width 0.25) (layer "B.Cu") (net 12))
 (segment (start 94.0054 72.3392) (end 92.6819 73.6627) (width 0.25) (layer "B.Cu") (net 11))
 (segment (start 92.6819 73.6627) (end 72.3954 73.6627) (width 0.25) (layer "B.Cu") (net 11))
 (segment (start 111.188 72.0725) (end 110.922 72.3392) (width 0.25) (layer "B.Cu") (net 11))
 (segment (start 110.922 72.3392) (end 94.0054 72.3392) (width 0.25) (layer "B.Cu") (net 11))
 (segment (start 122.694 102.744) (end 122.718 102.769) (width 0.25) (layer "F.Cu") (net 35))
 (segment (start 111.328 92.4306) (end 117.729 98.8314) (width 0.25) (layer "F.Cu") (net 35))
 (segment (start 122.743 102.794) (end 121.95 102.002) (width 0.25) (layer "F.Cu") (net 35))
 (segment (start 138.415 104.267) (end 137.24 104.267) (width 0.25) (layer "F.Cu") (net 35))
 (segment (start 95.23 86.3627) (end 98.4785 89.6112) (width 0.25) (layer "F.Cu") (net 35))
 (segment (start 121.158 101.209) (end 121.95 102.002) (width 0.25) (layer "F.Cu") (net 35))
 (segment (start 108.433 89.6112) (end 108.698 89.8763) (width 0.25) (layer "F.Cu") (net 35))
 (segment (start 137.24 104.267) (end 137.24 103.9) (width 0.25) (layer "F.Cu") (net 35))
 (segment (start 136.134 102.794) (end 122.743 102.794) (width 0.25) (layer "F.Cu") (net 35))
 (segment (start 121.95 102.002) (end 121.951 102.002) (width 0.25) (layer "F.Cu") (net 35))
 (segment (start 121.158 100.584) (end 121.158 101.209) (width 0.25) (layer "F.Cu") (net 35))
 (segment (start 137.24 103.9) (end 136.134 102.794) (width 0.25) (layer "F.Cu") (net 35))
 (segment (start 117.729 98.8314) (end 117.729 98.8822) (width 0.25) (layer "F.Cu") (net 35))
 (segment (start 98.4785 89.6112) (end 108.433 89.6112) (width 0.25) (layer "F.Cu") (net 35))
 (segment (start 122.644 102.695) (end 122.694 102.744) (width 0.25) (layer "F.Cu") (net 35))
 (segment (start 121.951 102.002) (end 122.644 102.695) (width 0.25) (layer "F.Cu") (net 35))
 (segment (start 122.718 102.769) (end 122.743 102.794) (width 0.25) (layer "F.Cu") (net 35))
 (via (at 108.698 89.8763) (size 0.8) (drill 0.4) (layers "F.Cu" "B.Cu") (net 35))
 (via (at 111.328 92.4306) (size 0.8) (drill 0.4) (layers "F.Cu" "B.Cu") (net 35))
 (via (at 117.729 98.8822) (size 0.8) (drill 0.4) (layers "F.Cu" "B.Cu") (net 35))
 (via (at 121.158 100.584) (size 0.8) (drill 0.4) (layers "F.Cu" "B.Cu") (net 35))
 (segment (start 111.252 92.4306) (end 111.328 92.4306) (width 0.25) (layer "B.Cu") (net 35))
 (segment (start 119.456 98.8822) (end 121.158 100.584) (width 0.25) (layer "B.Cu") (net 35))
 (segment (start 117.729 98.8822) (end 119.456 98.8822) (width 0.25) (layer "B.Cu") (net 35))
 (segment (start 108.698 89.8763) (end 111.252 92.4306) (width 0.25) (layer "B.Cu") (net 35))
 (segment (start 95.23 66.0427) (end 97.6376 68.4503) (width 0.25) (layer "F.Cu") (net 3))
 (segment (start 97.6376 68.4503) (end 97.6376 76.835) (width 0.25) (layer "F.Cu") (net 3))
 (via (at 97.6376 76.835) (size 0.8) (drill 0.4) (layers "F.Cu" "B.Cu") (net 3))
 (segment (start 99.9488 103.352) (end 100.435 103.839) (width 0.25) (layer "B.Cu") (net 3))
 (segment (start 99.9488 103.352) (end 100.436 103.839) (width 0.25) (layer "B.Cu") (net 3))
 (segment (start 100.889 103.839) (end 100.889 104.4095) (width 0.25) (layer "B.Cu") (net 3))
 (segment (start 97.6376 76.835) (end 97.6376 101.041) (width 0.25) (layer "B.Cu") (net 3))
 (segment (start 100.436 103.839) (end 100.889 103.839) (width 0.25) (layer "B.Cu") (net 3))
 (segment (start 97.6376 101.041) (end 99.9488 103.352) (width 0.25) (layer "B.Cu") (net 3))
 (segment (start 100.436 103.839) (end 102.26 105.664) (width 0.25) (layer "B.Cu") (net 3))
 (segment (start 100.435 103.839) (end 100.436 103.839) (width 0.25) (layer "B.Cu") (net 3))
 (segment (start 92.2274 74.93) (end 92.4052 74.7522) (width 0.25) (layer "F.Cu") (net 10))
 (segment (start 72.3954 60.9627) (end 84.7598 73.3271) (width 0.25) (layer "F.Cu") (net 10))
 (segment (start 84.7598 73.3271) (end 84.7598 74.93) (width 0.25) (layer "F.Cu") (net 10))
 (segment (start 84.7598 74.93) (end 92.2274 74.93) (width 0.25) (layer "F.Cu") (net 10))
 (via (at 92.4052 74.7522) (size 0.8) (drill 0.4) (layers "F.Cu" "B.Cu") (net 10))
 (segment (start 109.166 74.5969) (end 109.417 74.848) (width 0.25) (layer "B.Cu") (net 10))
 (segment (start 118.9355 75.273) (end 119.863 74.346) (width 0.25) (layer "B.Cu") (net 10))
 (segment (start 118.008 76.2) (end 118.9355 75.273) (width 0.25) (layer "B.Cu") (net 10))
 (segment (start 109.417 74.848) (end 109.92 75.3503) (width 0.25) (layer "B.Cu") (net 10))
 (segment (start 118.9355 75.273) (end 119.8626 74.3459) (width 0.25) (layer "B.Cu") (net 10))
 (segment (start 108.509 74.7522) (end 108.712 74.549) (width 0.25) (layer "B.Cu") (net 10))
 (segment (start 109.92 75.3503) (end 109.92 75.351) (width 0.25) (layer "B.Cu") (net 10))
 (segment (start 110.769 76.2) (end 118.008 76.2) (width 0.25) (layer "B.Cu") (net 10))
 (segment (start 109.92 75.351) (end 110.769 76.2) (width 0.25) (layer "B.Cu") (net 10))
 (segment (start 92.4052 74.7522) (end 108.509 74.7522) (width 0.25) (layer "B.Cu") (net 10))
 (segment (start 98.4121 66.6875) (end 98.4121 77.5905) (width 0.25) (layer "F.Cu") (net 40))
 (segment (start 95.23 63.5054) (end 98.4121 66.6875) (width 0.25) (layer "F.Cu") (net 40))
 (via (at 98.4121 77.5905) (size 0.8) (drill 0.4) (layers "F.Cu" "B.Cu") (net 40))
 (segment (start 99.949 79.1274) (end 99.949 81.2292) (width 0.25) (layer "B.Cu") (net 40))
 (segment (start 98.4121 77.5905) (end 99.949 79.1274) (width 0.25) (layer "B.Cu") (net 40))
 (segment (start 126.35 88.6101) (end 127.229 87.7316) (width 0.25) (layer "F.Cu") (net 7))
 (segment (start 109.904 82.8714) (end 115.643 88.6101) (width 0.25) (layer "F.Cu") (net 7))
 (segment (start 127.229 87.7316) (end 128.316 86.6445) (width 0.25) (layer "F.Cu") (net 7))
 (segment (start 115.643 88.6101) (end 126.35 88.6101) (width 0.25) (layer "F.Cu") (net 7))
 (segment (start 140.955 94.7973) (end 140.955 104.267) (width 0.25) (layer "F.Cu") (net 7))
 (segment (start 135.636 87.6554) (end 135.636 89.4783) (width 0.25) (layer "F.Cu") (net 7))
 (segment (start 104.784 82.8714) (end 109.904 82.8714) (width 0.25) (layer "F.Cu") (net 7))
 (segment (start 134.6251 86.6445) (end 135.636 87.6554) (width 0.25) (layer "F.Cu") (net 7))
 (segment (start 135.636 89.4783) (end 140.955 94.7973) (width 0.25) (layer "F.Cu") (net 7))
 (segment (start 128.316 86.6445) (end 134.6251 86.6445) (width 0.25) (layer "F.Cu") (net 7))
 (via (at 104.784 82.8714) (size 0.8) (drill 0.4) (layers "F.Cu" "B.Cu") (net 7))
 (segment (start 104.352 82.8714) (end 100.6169 86.6065) (width 0.25) (layer "B.Cu") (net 7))
 (segment (start 99.9236 86.6065) (end 99.9236 87.7316) (width 0.25) (layer "B.Cu") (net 7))
 (segment (start 100.6169 86.6065) (end 99.9236 86.6065) (width 0.25) (layer "B.Cu") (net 7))
 (segment (start 104.784 82.8714) (end 104.352 82.8714) (width 0.25) (layer "B.Cu") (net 7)))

